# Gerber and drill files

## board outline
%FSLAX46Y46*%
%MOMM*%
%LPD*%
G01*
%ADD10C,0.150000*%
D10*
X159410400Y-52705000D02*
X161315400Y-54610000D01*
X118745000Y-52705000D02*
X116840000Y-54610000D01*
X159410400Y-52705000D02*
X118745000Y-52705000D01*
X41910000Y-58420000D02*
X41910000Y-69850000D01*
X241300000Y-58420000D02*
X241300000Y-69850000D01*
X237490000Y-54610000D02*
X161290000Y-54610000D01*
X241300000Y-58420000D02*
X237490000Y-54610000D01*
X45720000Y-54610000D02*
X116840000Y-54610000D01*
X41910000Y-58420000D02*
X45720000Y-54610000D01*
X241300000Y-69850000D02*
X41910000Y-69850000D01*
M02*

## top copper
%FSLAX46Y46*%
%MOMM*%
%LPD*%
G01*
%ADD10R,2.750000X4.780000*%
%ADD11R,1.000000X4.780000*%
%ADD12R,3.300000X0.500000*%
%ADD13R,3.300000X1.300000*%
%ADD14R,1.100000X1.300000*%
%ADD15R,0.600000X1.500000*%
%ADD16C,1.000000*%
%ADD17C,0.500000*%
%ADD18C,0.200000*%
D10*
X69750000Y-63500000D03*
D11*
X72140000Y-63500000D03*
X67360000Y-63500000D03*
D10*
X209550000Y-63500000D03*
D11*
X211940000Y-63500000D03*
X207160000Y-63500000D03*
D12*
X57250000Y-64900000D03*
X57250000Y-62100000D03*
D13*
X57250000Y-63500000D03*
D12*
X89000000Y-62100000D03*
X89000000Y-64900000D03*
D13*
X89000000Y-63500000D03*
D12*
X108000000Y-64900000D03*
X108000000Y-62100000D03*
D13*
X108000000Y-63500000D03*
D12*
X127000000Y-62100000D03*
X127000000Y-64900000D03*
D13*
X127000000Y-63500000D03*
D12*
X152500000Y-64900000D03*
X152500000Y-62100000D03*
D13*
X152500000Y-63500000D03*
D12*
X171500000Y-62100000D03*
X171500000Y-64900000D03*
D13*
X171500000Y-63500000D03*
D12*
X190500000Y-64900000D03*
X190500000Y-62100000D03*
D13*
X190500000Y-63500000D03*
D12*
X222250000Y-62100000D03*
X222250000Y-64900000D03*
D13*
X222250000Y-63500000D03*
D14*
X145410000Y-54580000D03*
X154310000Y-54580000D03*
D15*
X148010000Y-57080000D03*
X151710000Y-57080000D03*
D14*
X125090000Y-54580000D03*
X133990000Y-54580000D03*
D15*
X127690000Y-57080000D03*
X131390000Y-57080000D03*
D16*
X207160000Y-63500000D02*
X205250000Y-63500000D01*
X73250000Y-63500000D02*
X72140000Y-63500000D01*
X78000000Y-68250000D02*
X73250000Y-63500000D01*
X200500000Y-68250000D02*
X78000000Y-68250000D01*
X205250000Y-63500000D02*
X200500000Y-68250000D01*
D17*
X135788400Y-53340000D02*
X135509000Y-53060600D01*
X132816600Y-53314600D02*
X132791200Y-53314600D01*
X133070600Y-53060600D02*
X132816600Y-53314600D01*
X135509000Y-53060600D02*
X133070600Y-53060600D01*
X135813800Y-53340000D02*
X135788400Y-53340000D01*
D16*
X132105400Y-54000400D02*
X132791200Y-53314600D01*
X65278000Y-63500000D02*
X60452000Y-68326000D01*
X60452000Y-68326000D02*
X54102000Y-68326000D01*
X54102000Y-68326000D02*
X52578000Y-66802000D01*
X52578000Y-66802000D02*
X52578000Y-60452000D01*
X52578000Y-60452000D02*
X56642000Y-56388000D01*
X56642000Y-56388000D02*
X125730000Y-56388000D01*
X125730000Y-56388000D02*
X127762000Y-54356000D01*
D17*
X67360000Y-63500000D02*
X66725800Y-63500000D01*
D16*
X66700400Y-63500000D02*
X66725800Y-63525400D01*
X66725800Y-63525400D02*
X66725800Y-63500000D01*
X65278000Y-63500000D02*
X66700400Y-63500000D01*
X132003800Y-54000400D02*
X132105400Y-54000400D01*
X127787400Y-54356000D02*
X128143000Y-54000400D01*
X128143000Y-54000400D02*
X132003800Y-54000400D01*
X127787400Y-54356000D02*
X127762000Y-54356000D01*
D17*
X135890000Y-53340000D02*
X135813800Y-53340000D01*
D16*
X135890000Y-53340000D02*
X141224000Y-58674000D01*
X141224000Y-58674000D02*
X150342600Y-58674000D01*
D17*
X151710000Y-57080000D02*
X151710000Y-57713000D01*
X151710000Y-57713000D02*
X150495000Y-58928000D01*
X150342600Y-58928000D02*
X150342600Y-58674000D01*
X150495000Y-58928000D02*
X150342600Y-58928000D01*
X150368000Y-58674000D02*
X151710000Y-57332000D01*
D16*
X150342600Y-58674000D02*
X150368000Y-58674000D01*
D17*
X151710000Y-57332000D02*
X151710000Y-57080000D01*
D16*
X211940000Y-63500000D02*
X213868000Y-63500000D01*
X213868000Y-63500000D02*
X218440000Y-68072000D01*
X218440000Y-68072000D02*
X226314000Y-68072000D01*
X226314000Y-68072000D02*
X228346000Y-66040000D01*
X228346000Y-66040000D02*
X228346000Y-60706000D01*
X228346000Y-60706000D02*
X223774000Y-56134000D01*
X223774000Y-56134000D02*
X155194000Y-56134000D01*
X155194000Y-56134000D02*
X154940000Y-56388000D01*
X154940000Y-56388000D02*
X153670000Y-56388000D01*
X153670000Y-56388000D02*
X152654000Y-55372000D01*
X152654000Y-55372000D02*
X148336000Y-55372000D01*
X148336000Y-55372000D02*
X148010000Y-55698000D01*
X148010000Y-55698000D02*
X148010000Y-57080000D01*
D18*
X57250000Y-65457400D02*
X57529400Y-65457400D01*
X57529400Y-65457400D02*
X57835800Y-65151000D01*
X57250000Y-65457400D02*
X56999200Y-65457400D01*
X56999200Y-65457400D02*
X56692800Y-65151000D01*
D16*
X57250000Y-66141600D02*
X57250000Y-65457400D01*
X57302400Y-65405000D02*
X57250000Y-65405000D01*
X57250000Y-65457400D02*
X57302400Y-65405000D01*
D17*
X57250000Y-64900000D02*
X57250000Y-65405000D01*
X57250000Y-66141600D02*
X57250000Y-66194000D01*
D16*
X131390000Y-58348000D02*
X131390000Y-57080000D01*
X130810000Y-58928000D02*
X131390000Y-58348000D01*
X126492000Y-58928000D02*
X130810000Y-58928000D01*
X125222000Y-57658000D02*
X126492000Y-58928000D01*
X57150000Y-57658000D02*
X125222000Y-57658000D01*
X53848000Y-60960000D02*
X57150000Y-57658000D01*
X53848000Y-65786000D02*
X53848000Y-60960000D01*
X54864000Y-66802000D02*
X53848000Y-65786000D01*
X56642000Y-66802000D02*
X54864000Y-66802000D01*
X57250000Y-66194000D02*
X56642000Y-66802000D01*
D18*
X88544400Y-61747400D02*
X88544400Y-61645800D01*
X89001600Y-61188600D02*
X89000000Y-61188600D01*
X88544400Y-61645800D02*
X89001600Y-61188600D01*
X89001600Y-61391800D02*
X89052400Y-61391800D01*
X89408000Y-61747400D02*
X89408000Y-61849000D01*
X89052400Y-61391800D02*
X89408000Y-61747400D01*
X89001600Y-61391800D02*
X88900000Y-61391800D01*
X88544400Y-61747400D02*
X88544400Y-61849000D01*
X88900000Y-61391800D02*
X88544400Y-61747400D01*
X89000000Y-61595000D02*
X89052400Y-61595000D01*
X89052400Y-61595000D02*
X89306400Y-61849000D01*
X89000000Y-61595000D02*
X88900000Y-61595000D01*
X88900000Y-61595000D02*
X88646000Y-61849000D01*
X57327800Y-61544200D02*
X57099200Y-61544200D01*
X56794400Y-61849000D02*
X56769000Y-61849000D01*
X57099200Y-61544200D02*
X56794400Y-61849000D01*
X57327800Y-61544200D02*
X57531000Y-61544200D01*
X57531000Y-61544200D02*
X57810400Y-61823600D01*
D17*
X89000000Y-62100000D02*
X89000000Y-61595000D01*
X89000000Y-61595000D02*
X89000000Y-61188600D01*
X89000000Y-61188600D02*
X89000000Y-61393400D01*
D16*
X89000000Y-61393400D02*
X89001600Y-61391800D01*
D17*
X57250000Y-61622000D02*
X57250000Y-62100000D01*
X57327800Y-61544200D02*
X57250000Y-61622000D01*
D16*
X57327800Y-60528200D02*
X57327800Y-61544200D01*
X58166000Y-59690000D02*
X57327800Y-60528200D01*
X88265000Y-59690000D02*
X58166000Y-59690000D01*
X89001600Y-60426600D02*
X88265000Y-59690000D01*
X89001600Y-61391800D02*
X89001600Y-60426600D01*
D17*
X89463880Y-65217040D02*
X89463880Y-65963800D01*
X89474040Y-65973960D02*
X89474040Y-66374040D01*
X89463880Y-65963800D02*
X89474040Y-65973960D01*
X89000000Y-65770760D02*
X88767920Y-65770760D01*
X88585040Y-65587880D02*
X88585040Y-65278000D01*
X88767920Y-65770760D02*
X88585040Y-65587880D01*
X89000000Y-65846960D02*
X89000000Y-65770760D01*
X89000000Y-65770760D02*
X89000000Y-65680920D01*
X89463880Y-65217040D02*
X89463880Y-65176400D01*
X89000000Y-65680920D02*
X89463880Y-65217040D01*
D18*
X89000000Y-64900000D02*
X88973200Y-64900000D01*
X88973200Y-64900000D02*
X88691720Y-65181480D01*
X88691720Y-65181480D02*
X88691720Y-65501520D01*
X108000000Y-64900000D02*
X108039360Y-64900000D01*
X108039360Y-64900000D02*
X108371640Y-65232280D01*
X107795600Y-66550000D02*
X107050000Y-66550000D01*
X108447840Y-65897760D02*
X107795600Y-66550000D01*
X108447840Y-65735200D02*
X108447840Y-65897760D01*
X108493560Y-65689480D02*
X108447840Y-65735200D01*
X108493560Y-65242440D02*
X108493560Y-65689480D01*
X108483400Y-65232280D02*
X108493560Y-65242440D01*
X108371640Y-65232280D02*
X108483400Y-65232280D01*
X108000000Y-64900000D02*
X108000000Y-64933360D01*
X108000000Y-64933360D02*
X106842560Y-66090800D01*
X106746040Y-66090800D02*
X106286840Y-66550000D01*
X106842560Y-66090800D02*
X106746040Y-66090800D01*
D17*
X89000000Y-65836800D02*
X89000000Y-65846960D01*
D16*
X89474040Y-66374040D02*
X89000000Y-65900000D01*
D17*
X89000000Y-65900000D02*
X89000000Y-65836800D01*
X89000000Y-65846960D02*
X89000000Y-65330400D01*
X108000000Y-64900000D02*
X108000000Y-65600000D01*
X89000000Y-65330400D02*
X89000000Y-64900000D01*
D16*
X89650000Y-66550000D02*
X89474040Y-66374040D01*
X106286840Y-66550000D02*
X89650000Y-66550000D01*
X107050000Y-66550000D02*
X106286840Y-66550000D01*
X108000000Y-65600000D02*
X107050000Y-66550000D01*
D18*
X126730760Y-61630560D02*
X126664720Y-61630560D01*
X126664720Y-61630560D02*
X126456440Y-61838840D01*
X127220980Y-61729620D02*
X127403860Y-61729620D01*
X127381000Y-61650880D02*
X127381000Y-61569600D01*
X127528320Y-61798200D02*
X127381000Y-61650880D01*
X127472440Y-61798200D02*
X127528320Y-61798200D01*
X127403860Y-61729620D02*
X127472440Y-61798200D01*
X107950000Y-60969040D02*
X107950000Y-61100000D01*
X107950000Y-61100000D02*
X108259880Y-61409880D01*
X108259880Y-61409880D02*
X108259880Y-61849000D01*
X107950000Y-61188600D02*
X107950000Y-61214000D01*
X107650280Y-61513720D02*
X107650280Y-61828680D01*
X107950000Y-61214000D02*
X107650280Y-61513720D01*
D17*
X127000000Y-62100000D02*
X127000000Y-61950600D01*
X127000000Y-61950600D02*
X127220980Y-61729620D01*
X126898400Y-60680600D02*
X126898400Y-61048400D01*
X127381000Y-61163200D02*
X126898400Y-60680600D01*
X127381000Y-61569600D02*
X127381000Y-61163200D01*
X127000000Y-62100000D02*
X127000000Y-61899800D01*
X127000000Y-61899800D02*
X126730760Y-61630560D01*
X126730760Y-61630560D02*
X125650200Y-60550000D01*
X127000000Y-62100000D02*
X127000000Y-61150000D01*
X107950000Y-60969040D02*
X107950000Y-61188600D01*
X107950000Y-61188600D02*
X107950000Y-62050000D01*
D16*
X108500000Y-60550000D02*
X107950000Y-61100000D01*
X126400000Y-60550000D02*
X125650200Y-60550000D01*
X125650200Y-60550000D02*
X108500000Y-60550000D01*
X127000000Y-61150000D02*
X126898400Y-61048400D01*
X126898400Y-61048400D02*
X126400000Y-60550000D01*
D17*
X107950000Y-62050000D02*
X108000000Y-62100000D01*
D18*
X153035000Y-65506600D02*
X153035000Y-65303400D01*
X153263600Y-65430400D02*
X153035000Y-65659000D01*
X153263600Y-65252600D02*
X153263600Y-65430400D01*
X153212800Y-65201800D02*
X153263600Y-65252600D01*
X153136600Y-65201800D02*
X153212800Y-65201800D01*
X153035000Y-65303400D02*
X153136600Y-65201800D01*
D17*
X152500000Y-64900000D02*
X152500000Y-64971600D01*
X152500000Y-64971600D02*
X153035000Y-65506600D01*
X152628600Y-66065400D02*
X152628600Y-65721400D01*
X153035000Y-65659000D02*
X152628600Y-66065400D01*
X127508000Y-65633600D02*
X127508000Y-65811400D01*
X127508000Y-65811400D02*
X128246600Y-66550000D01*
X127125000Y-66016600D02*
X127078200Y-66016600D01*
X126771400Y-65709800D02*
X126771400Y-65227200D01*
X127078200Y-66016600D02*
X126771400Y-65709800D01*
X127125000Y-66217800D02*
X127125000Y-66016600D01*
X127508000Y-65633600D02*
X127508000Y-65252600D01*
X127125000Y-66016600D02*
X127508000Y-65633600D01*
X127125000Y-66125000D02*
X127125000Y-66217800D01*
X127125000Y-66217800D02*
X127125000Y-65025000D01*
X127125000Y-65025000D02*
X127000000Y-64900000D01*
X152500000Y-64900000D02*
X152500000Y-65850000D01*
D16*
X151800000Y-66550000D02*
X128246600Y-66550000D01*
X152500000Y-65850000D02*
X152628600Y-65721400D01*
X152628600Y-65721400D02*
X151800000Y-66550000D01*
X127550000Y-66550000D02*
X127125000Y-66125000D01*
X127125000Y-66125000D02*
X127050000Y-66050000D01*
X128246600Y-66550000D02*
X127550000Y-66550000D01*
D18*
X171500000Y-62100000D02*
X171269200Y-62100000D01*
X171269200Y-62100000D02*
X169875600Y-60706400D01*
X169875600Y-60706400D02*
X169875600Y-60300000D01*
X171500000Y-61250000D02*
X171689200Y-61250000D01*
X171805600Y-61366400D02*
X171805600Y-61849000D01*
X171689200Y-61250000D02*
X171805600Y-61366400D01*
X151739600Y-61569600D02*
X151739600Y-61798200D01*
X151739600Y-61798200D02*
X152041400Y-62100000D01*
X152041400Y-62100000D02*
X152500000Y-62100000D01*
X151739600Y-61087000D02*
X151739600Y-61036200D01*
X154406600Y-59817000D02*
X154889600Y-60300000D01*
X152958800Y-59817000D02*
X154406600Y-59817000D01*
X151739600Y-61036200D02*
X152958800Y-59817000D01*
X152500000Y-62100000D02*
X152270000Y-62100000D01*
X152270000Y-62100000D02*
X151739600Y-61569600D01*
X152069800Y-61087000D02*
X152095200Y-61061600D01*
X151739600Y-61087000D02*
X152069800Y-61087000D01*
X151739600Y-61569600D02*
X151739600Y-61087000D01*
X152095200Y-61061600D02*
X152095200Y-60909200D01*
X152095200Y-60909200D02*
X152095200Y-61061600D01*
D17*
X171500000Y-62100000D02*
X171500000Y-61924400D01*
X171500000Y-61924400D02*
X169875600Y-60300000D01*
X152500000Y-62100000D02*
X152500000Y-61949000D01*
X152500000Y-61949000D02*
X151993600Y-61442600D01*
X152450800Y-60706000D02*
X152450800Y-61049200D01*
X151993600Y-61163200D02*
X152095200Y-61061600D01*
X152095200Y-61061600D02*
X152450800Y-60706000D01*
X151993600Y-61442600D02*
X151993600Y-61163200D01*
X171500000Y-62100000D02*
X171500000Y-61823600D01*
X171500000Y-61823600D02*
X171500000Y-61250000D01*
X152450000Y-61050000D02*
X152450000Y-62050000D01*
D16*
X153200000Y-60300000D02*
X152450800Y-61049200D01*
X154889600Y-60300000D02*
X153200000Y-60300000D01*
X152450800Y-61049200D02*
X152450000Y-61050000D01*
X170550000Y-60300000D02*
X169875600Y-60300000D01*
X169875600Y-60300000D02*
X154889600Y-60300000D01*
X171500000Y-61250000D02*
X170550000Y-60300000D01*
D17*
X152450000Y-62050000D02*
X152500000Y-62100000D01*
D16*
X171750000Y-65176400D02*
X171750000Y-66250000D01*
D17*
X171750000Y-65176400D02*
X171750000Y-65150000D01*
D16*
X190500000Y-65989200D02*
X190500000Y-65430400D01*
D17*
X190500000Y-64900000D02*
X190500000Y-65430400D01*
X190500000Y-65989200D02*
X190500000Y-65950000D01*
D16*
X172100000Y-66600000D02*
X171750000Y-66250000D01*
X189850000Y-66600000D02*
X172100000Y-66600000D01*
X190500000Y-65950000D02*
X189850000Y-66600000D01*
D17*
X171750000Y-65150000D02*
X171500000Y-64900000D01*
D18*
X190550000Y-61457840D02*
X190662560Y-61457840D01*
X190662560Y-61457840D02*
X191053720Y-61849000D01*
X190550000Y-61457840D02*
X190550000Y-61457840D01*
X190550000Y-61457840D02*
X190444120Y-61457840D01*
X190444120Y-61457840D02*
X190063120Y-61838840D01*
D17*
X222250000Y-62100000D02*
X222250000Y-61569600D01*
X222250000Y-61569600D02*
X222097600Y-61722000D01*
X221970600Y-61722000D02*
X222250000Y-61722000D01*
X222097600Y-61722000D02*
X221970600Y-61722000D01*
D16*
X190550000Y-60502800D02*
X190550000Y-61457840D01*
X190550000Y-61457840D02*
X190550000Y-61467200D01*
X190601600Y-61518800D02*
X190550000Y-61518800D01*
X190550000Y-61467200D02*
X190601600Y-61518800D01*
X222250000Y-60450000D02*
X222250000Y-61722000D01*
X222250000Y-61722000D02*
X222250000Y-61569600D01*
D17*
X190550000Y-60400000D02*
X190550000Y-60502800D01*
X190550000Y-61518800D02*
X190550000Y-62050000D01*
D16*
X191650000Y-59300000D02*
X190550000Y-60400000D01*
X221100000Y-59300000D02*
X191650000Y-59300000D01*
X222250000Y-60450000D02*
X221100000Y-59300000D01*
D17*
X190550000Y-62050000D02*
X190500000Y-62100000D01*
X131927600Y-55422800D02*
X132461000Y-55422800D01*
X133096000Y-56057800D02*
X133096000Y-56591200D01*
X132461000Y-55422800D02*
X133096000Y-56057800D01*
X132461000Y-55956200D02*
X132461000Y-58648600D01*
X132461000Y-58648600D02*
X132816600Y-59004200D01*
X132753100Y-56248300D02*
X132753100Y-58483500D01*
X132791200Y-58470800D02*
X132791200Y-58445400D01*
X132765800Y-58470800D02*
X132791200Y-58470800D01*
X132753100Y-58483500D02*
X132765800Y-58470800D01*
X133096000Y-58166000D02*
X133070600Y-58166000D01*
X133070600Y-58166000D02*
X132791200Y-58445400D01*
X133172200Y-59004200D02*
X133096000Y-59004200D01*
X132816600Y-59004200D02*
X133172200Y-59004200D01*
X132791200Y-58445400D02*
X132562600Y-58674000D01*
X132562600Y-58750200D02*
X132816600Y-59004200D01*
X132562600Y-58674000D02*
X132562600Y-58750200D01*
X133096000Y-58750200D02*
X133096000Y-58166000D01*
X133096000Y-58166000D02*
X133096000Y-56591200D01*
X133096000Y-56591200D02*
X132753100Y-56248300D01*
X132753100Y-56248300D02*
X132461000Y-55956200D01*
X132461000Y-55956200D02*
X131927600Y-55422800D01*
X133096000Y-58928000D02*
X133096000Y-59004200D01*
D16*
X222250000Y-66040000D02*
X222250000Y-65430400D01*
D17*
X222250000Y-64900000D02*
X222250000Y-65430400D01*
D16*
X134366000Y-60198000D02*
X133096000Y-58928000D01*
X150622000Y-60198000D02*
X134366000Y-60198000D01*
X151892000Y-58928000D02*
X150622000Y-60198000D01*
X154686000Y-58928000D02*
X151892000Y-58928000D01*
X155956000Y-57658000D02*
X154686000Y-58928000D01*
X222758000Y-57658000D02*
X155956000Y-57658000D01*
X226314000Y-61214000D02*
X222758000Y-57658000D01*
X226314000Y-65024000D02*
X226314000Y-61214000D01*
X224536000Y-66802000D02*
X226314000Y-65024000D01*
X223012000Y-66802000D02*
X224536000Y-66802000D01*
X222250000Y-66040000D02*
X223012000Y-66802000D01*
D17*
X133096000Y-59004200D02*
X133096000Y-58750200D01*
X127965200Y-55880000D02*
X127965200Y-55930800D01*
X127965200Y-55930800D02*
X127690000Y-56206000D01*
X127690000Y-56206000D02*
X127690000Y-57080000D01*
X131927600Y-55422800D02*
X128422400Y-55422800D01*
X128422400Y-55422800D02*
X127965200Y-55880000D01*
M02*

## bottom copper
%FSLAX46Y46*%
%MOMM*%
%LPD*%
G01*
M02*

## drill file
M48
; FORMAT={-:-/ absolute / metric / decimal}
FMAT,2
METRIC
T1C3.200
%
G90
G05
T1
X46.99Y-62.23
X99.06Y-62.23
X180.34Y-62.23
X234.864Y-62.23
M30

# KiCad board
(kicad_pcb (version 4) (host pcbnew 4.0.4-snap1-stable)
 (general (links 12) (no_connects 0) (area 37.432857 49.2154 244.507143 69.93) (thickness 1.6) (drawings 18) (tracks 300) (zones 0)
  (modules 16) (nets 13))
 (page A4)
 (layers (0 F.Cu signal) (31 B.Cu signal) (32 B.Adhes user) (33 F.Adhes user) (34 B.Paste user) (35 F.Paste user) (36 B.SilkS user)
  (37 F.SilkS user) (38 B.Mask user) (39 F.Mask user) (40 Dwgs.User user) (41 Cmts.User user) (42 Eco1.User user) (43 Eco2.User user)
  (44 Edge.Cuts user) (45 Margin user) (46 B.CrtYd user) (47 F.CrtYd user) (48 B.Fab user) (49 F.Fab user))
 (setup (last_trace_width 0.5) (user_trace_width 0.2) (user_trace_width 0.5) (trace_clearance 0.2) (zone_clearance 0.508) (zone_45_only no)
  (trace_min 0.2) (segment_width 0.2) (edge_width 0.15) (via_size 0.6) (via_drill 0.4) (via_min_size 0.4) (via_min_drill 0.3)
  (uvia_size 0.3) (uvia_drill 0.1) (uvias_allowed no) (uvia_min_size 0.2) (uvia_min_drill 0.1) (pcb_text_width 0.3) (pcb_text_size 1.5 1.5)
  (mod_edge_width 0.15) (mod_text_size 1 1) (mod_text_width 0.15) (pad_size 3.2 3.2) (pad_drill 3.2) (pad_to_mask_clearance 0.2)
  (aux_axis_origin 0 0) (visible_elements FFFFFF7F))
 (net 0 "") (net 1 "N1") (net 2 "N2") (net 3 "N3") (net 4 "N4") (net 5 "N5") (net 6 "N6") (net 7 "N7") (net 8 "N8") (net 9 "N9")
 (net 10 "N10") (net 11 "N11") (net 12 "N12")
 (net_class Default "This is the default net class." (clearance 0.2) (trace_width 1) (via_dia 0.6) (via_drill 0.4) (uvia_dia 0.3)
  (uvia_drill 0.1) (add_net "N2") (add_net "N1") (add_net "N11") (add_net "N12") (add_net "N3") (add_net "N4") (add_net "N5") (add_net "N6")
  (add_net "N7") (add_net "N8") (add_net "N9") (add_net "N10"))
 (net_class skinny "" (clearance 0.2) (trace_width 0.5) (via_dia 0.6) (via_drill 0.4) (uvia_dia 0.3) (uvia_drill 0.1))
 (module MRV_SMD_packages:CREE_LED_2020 (layer F.Cu) (at 69.75 63.5 180)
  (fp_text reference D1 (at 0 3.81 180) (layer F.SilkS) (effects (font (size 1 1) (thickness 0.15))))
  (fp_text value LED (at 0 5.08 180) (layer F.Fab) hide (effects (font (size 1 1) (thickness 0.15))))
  (pad 0 smd rect (at 0 0 180) (size 2.75 4.78) (layers F.Cu F.Mask) (solder_mask_margin -5))
  (pad 2 smd rect (at -2.39 0 180) (size 1 4.78) (layers F.Cu F.Paste F.Mask) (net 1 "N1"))
  (pad 1 smd rect (at 2.39 0 180) (size 1 4.78) (layers F.Cu F.Paste F.Mask) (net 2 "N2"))
  (pad 0 smd rect (at -0.61 -0.525 180) (size 0.97 0.8) (layers F.Paste F.Mask))
  (pad 0 smd rect (at -0.61 -1.575 180) (size 0.97 0.8) (layers F.Paste F.Mask))
  (pad 0 smd rect (at 0.61 -1.575 180) (size 0.97 0.8) (layers F.Paste F.Mask))
  (pad 0 smd rect (at 0.61 -0.525 180) (size 0.97 0.8) (layers F.Paste F.Mask))
  (pad 0 smd rect (at 0.61 0.525 180) (size 0.97 0.8) (layers F.Paste F.Mask))
  (pad 0 smd rect (at -0.61 0.525 180) (size 0.97 0.8) (layers F.Paste F.Mask))
  (pad 0 smd rect (at -0.61 1.575 180) (size 0.97 0.8) (layers F.Paste F.Mask))
  (pad 0 smd rect (at 0.61 1.575 180) (size 0.97 0.8) (layers F.Paste F.Mask)))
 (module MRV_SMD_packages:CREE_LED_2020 (layer F.Cu) (at 209.55 63.5 180)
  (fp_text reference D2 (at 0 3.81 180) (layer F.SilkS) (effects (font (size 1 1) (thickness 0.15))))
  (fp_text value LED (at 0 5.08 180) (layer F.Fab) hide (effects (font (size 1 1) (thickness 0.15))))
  (pad 0 smd rect (at 0 0 180) (size 2.75 4.78) (layers F.Cu F.Mask) (solder_mask_margin -5))
  (pad 2 smd rect (at -2.39 0 180) (size 1 4.78) (layers F.Cu F.Paste F.Mask) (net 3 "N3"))
  (pad 1 smd rect (at 2.39 0 180) (size 1 4.78) (layers F.Cu F.Paste F.Mask) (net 1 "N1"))
  (pad 0 smd rect (at -0.61 -0.525 180) (size 0.97 0.8) (layers F.Paste F.Mask))
  (pad 0 smd rect (at -0.61 -1.575 180) (size 0.97 0.8) (layers F.Paste F.Mask))
  (pad 0 smd rect (at 0.61 -1.575 180) (size 0.97 0.8) (layers F.Paste F.Mask))
  (pad 0 smd rect (at 0.61 -0.525 180) (size 0.97 0.8) (layers F.Paste F.Mask))
  (pad 0 smd rect (at 0.61 0.525 180) (size 0.97 0.8) (layers F.Paste F.Mask))
  (pad 0 smd rect (at -0.61 0.525 180) (size 0.97 0.8) (layers F.Paste F.Mask))
  (pad 0 smd rect (at -0.61 1.575 180) (size 0.97 0.8) (layers F.Paste F.Mask))
  (pad 0 smd rect (at 0.61 1.575 180) (size 0.97 0.8) (layers F.Paste F.Mask)))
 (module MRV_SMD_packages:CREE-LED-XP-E (layer F.Cu) (at 57.25 63.5 270)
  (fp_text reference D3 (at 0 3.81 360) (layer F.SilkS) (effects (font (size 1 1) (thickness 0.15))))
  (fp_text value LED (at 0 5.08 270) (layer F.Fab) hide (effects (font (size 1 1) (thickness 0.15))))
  (pad 1 smd rect (at 1.4 0 270) (size 0.5 3.3) (layers F.Cu F.Paste F.Mask) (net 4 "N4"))
  (pad 2 smd rect (at -1.4 0 270) (size 0.5 3.3) (layers F.Cu F.Paste F.Mask) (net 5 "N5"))
  (pad 0 smd rect (at 0 0 270) (size 1.3 3.3) (layers F.Cu F.Paste F.Mask)))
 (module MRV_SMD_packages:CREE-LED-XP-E (layer F.Cu) (at 89 63.5 90)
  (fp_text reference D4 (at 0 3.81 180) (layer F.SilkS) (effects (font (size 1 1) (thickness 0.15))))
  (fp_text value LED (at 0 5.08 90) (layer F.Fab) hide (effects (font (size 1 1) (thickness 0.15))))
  (pad 1 smd rect (at 1.4 0 90) (size 0.5 3.3) (layers F.Cu F.Paste F.Mask) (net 5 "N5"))
  (pad 2 smd rect (at -1.4 0 90) (size 0.5 3.3) (layers F.Cu F.Paste F.Mask) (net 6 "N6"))
  (pad 0 smd rect (at 0 0 90) (size 1.3 3.3) (layers F.Cu F.Paste F.Mask)))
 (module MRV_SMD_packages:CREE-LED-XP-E (layer F.Cu) (at 108 63.5 270)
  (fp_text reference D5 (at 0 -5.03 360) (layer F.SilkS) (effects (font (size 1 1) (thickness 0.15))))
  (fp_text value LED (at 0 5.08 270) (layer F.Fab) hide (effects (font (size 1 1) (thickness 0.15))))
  (pad 1 smd rect (at 1.4 0 270) (size 0.5 3.3) (layers F.Cu F.Paste F.Mask) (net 6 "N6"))
  (pad 2 smd rect (at -1.4 0 270) (size 0.5 3.3) (layers F.Cu F.Paste F.Mask) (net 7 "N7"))
  (pad 0 smd rect (at 0 0 270) (size 1.3 3.3) (layers F.Cu F.Paste F.Mask)))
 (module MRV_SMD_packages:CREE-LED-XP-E (layer F.Cu) (at 127 63.5 90)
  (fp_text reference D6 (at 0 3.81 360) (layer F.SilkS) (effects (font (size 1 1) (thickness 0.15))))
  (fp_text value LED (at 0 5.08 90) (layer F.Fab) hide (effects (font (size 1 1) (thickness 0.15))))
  (pad 1 smd rect (at 1.4 0 90) (size 0.5 3.3) (layers F.Cu F.Paste F.Mask) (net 7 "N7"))
  (pad 2 smd rect (at -1.4 0 90) (size 0.5 3.3) (layers F.Cu F.Paste F.Mask) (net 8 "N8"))
  (pad 0 smd rect (at 0 0 90) (size 1.3 3.3) (layers F.Cu F.Paste F.Mask)))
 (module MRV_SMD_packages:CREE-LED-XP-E (layer F.Cu) (at 152.5 63.5 270)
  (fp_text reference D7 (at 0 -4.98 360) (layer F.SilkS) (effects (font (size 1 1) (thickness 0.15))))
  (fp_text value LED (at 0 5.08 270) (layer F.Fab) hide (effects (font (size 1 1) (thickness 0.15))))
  (pad 1 smd rect (at 1.4 0 270) (size 0.5 3.3) (layers F.Cu F.Paste F.Mask) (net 8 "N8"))
  (pad 2 smd rect (at -1.4 0 270) (size 0.5 3.3) (layers F.Cu F.Paste F.Mask) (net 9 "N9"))
  (pad 0 smd rect (at 0 0 270) (size 1.3 3.3) (layers F.Cu F.Paste F.Mask)))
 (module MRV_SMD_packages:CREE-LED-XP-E (layer F.Cu) (at 171.5 63.5 90)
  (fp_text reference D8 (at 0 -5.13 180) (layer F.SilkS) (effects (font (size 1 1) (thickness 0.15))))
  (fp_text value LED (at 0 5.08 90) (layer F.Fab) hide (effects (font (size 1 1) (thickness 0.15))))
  (pad 1 smd rect (at 1.4 0 90) (size 0.5 3.3) (layers F.Cu F.Paste F.Mask) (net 9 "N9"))
  (pad 2 smd rect (at -1.4 0 90) (size 0.5 3.3) (layers F.Cu F.Paste F.Mask) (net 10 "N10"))
  (pad 0 smd rect (at 0 0 90) (size 1.3 3.3) (layers F.Cu F.Paste F.Mask)))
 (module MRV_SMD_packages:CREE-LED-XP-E (layer F.Cu) (at 190.5 63.5 270)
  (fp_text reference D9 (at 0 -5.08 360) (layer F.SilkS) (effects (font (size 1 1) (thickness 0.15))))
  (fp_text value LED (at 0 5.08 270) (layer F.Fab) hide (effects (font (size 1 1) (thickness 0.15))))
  (pad 1 smd rect (at 1.4 0 270) (size 0.5 3.3) (layers F.Cu F.Paste F.Mask) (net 10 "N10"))
  (pad 2 smd rect (at -1.4 0 270) (size 0.5 3.3) (layers F.Cu F.Paste F.Mask) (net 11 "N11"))
  (pad 0 smd rect (at 0 0 270) (size 1.3 3.3) (layers F.Cu F.Paste F.Mask)))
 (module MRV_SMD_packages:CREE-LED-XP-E (layer F.Cu) (at 222.25 63.5 90)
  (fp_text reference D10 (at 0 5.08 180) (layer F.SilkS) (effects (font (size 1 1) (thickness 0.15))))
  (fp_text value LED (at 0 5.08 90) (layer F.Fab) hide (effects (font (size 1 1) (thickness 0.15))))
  (pad 1 smd rect (at 1.4 0 90) (size 0.5 3.3) (layers F.Cu F.Paste F.Mask) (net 11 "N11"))
  (pad 2 smd rect (at -1.4 0 90) (size 0.5 3.3) (layers F.Cu F.Paste F.Mask) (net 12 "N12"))
  (pad 0 smd rect (at 0 0 90) (size 1.3 3.3) (layers F.Cu F.Paste F.Mask)))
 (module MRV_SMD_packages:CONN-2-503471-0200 (layer F.Cu) (at 149.86 55.88 180)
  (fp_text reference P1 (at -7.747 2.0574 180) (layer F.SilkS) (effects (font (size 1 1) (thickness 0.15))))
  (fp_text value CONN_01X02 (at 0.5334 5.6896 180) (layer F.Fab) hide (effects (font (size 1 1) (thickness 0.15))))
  (pad 0 smd rect (at 4.45 1.3 180) (size 1.1 1.3) (layers F.Cu F.Paste F.Mask))
  (pad 0 smd rect (at -4.45 1.3 180) (size 1.1 1.3) (layers F.Cu F.Paste F.Mask))
  (pad 2 smd rect (at 1.85 -1.2 180) (size 0.6 1.5) (layers F.Cu F.Paste F.Mask) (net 3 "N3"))
  (pad 1 smd rect (at -1.85 -1.2 180) (size 0.6 1.5) (layers F.Cu F.Paste F.Mask) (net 2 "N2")))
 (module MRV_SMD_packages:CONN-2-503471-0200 (layer F.Cu) (at 129.54 55.88 180)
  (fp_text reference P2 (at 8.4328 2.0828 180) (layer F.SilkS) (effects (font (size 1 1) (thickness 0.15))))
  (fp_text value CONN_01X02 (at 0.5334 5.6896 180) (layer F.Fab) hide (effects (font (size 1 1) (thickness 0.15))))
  (pad 0 smd rect (at 4.45 1.3 180) (size 1.1 1.3) (layers F.Cu F.Paste F.Mask))
  (pad 0 smd rect (at -4.45 1.3 180) (size 1.1 1.3) (layers F.Cu F.Paste F.Mask))
  (pad 2 smd rect (at 1.85 -1.2 180) (size 0.6 1.5) (layers F.Cu F.Paste F.Mask) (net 12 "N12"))
  (pad 1 smd rect (at -1.85 -1.2 180) (size 0.6 1.5) (layers F.Cu F.Paste F.Mask) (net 4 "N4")))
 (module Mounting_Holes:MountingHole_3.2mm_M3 (layer F.Cu) (at 46.99 62.23)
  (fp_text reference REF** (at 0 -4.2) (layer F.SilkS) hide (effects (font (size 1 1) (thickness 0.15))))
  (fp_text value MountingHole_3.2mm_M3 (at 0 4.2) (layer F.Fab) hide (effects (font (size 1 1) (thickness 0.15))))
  (pad 1 np_thru_hole circle (at 0 0) (size 3.2 3.2) (drill 3.2) (layers *.Cu *.Mask F.SilkS)))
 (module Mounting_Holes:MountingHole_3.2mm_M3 (layer F.Cu) (at 234.86364 62.3062)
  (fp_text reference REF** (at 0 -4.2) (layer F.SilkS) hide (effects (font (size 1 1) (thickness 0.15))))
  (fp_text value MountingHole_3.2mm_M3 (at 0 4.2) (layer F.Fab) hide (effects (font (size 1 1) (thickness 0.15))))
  (pad "" np_thru_hole circle (at 0 -0.0762) (size 3.2 3.2) (drill 3.2) (layers *.Cu *.Mask F.SilkS)))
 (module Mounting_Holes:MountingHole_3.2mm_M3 (layer F.Cu) (at 180.34 62.23)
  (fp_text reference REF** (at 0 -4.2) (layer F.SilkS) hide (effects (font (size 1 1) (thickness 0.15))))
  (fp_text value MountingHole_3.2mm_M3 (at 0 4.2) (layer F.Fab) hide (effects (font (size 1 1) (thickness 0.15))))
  (pad 1 np_thru_hole circle (at 0 0) (size 3.2 3.2) (drill 3.2) (layers *.Cu *.Mask F.SilkS)))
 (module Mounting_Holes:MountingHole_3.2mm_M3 (layer F.Cu) (at 99.06 62.23)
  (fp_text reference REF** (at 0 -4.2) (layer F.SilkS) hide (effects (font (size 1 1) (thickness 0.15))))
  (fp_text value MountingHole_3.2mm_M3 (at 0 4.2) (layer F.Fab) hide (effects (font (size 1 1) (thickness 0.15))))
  (pad 1 np_thru_hole circle (at 0 0) (size 3.2 3.2) (drill 3.2) (layers *.Cu *.Mask F.SilkS)))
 (gr_line (start 159.4104 52.705) (end 161.3154 54.61) (angle 90) (layer Edge.Cuts) (width 0.15))
 (gr_line (start 118.745 52.705) (end 116.84 54.61) (angle 90) (layer Edge.Cuts) (width 0.15))
 (gr_line (start 159.4104 52.705) (end 118.745 52.705) (angle 90) (layer Edge.Cuts) (width 0.15))
 (gr_line (start 41.91 58.42) (end 41.91 69.85) (angle 90) (layer Edge.Cuts) (width 0.15))
 (gr_line (start 241.3 58.42) (end 241.3 69.85) (angle 90) (layer Edge.Cuts) (width 0.15))
 (gr_line (start 237.49 54.61) (end 161.29 54.61) (angle 90) (layer Edge.Cuts) (width 0.15))
 (gr_line (start 241.3 58.42) (end 237.49 54.61) (angle 90) (layer Edge.Cuts) (width 0.15))
 (gr_line (start 45.72 54.61) (end 116.84 54.61) (angle 90) (layer Edge.Cuts) (width 0.15))
 (gr_line (start 41.91 58.42) (end 45.72 54.61) (angle 90) (layer Edge.Cuts) (width 0.15))
 (gr_line (start 241.3 69.85) (end 41.91 69.85) (angle 90) (layer Edge.Cuts) (width 0.15))
 (segment (start 207.16 63.5) (end 205.25 63.5) (width 1) (layer F.Cu) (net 1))
 (segment (start 73.25 63.5) (end 72.14 63.5) (width 1) (layer F.Cu) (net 1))
 (segment (start 78 68.25) (end 73.25 63.5) (width 1) (layer F.Cu) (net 1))
 (segment (start 200.5 68.25) (end 78 68.25) (width 1) (layer F.Cu) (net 1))
 (segment (start 205.25 63.5) (end 200.5 68.25) (width 1) (layer F.Cu) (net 1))
 (segment (start 135.7884 53.34) (end 135.509 53.0606) (width 0.5) (layer F.Cu) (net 2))
 (segment (start 132.8166 53.3146) (end 132.7912 53.3146) (width 0.5) (layer F.Cu) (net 2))
 (segment (start 133.0706 53.0606) (end 132.8166 53.3146) (width 0.5) (layer F.Cu) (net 2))
 (segment (start 135.509 53.0606) (end 133.0706 53.0606) (width 0.5) (layer F.Cu) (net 2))
 (segment (start 135.8138 53.34) (end 135.7884 53.34) (width 0.5) (layer F.Cu) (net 2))
 (segment (start 132.1054 54.0004) (end 132.7912 53.3146) (width 1) (layer F.Cu) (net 2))
 (segment (start 65.278 63.5) (end 60.452 68.326) (width 1) (layer F.Cu) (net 2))
 (segment (start 60.452 68.326) (end 54.102 68.326) (width 1) (layer F.Cu) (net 2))
 (segment (start 54.102 68.326) (end 52.578 66.802) (width 1) (layer F.Cu) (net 2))
 (segment (start 52.578 66.802) (end 52.578 60.452) (width 1) (layer F.Cu) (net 2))
 (segment (start 52.578 60.452) (end 56.642 56.388) (width 1) (layer F.Cu) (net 2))
 (segment (start 56.642 56.388) (end 125.73 56.388) (width 1) (layer F.Cu) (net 2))
 (segment (start 125.73 56.388) (end 127.762 54.356) (width 1) (layer F.Cu) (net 2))
 (segment (start 67.36 63.5) (end 66.7258 63.5) (width 0.5) (layer F.Cu) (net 2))
 (segment (start 66.7004 63.5) (end 66.7258 63.5254) (width 1) (layer F.Cu) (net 2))
 (segment (start 66.7258 63.5254) (end 66.7258 63.5) (width 1) (layer F.Cu) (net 2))
 (segment (start 65.278 63.5) (end 66.7004 63.5) (width 1) (layer F.Cu) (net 2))
 (segment (start 132.0038 54.0004) (end 132.1054 54.0004) (width 1) (layer F.Cu) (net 2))
 (segment (start 127.7874 54.356) (end 128.143 54.0004) (width 1) (layer F.Cu) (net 2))
 (segment (start 128.143 54.0004) (end 132.0038 54.0004) (width 1) (layer F.Cu) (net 2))
 (segment (start 127.7874 54.356) (end 127.762 54.356) (width 1) (layer F.Cu) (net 2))
 (segment (start 135.89 53.34) (end 135.8138 53.34) (width 0.5) (layer F.Cu) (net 2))
 (segment (start 135.89 53.34) (end 141.224 58.674) (width 1) (layer F.Cu) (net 2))
 (segment (start 141.224 58.674) (end 150.3426 58.674) (width 1) (layer F.Cu) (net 2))
 (segment (start 151.71 57.08) (end 151.71 57.713) (width 0.5) (layer F.Cu) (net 2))
 (segment (start 151.71 57.713) (end 150.495 58.928) (width 0.5) (layer F.Cu) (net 2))
 (segment (start 150.3426 58.928) (end 150.3426 58.674) (width 0.5) (layer F.Cu) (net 2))
 (segment (start 150.495 58.928) (end 150.3426 58.928) (width 0.5) (layer F.Cu) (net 2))
 (segment (start 150.368 58.674) (end 151.71 57.332) (width 0.5) (layer F.Cu) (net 2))
 (segment (start 150.3426 58.674) (end 150.368 58.674) (width 1) (layer F.Cu) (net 2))
 (segment (start 151.71 57.332) (end 151.71 57.08) (width 0.5) (layer F.Cu) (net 2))
 (segment (start 211.94 63.5) (end 213.868 63.5) (width 1) (layer F.Cu) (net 3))
 (segment (start 213.868 63.5) (end 218.44 68.072) (width 1) (layer F.Cu) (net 3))
 (segment (start 218.44 68.072) (end 226.314 68.072) (width 1) (layer F.Cu) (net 3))
 (segment (start 226.314 68.072) (end 228.346 66.04) (width 1) (layer F.Cu) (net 3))
 (segment (start 228.346 66.04) (end 228.346 60.706) (width 1) (layer F.Cu) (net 3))
 (segment (start 228.346 60.706) (end 223.774 56.134) (width 1) (layer F.Cu) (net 3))
 (segment (start 223.774 56.134) (end 155.194 56.134) (width 1) (layer F.Cu) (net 3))
 (segment (start 155.194 56.134) (end 154.94 56.388) (width 1) (layer F.Cu) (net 3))
 (segment (start 154.94 56.388) (end 153.67 56.388) (width 1) (layer F.Cu) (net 3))
 (segment (start 153.67 56.388) (end 152.654 55.372) (width 1) (layer F.Cu) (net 3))
 (segment (start 152.654 55.372) (end 148.336 55.372) (width 1) (layer F.Cu) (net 3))
 (segment (start 148.336 55.372) (end 148.01 55.698) (width 1) (layer F.Cu) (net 3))
 (segment (start 148.01 55.698) (end 148.01 57.08) (width 1) (layer F.Cu) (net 3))
 (segment (start 57.25 65.4574) (end 57.5294 65.4574) (width 0.2) (layer F.Cu) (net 4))
 (segment (start 57.5294 65.4574) (end 57.8358 65.151) (width 0.2) (layer F.Cu) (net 4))
 (segment (start 57.25 65.4574) (end 56.9992 65.4574) (width 0.2) (layer F.Cu) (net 4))
 (segment (start 56.9992 65.4574) (end 56.6928 65.151) (width 0.2) (layer F.Cu) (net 4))
 (segment (start 57.25 66.1416) (end 57.25 65.4574) (width 1) (layer F.Cu) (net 4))
 (segment (start 57.3024 65.405) (end 57.25 65.405) (width 1) (layer F.Cu) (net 4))
 (segment (start 57.25 65.4574) (end 57.3024 65.405) (width 1) (layer F.Cu) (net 4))
 (segment (start 57.25 64.9) (end 57.25 65.405) (width 0.5) (layer F.Cu) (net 4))
 (segment (start 57.25 66.1416) (end 57.25 66.194) (width 0.5) (layer F.Cu) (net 4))
 (segment (start 131.39 58.348) (end 131.39 57.08) (width 1) (layer F.Cu) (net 4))
 (segment (start 130.81 58.928) (end 131.39 58.348) (width 1) (layer F.Cu) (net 4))
 (segment (start 126.492 58.928) (end 130.81 58.928) (width 1) (layer F.Cu) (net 4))
 (segment (start 125.222 57.658) (end 126.492 58.928) (width 1) (layer F.Cu) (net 4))
 (segment (start 57.15 57.658) (end 125.222 57.658) (width 1) (layer F.Cu) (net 4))
 (segment (start 53.848 60.96) (end 57.15 57.658) (width 1) (layer F.Cu) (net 4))
 (segment (start 53.848 65.786) (end 53.848 60.96) (width 1) (layer F.Cu) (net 4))
 (segment (start 54.864 66.802) (end 53.848 65.786) (width 1) (layer F.Cu) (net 4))
 (segment (start 56.642 66.802) (end 54.864 66.802) (width 1) (layer F.Cu) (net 4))
 (segment (start 57.25 66.194) (end 56.642 66.802) (width 1) (layer F.Cu) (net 4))
 (segment (start 88.5444 61.7474) (end 88.5444 61.6458) (width 0.2) (layer F.Cu) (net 5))
 (segment (start 89.0016 61.1886) (end 89 61.1886) (width 0.2) (layer F.Cu) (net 5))
 (segment (start 88.5444 61.6458) (end 89.0016 61.1886) (width 0.2) (layer F.Cu) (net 5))
 (segment (start 89.0016 61.3918) (end 89.0524 61.3918) (width 0.2) (layer F.Cu) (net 5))
 (segment (start 89.408 61.7474) (end 89.408 61.849) (width 0.2) (layer F.Cu) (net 5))
 (segment (start 89.0524 61.3918) (end 89.408 61.7474) (width 0.2) (layer F.Cu) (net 5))
 (segment (start 89.0016 61.3918) (end 88.9 61.3918) (width 0.2) (layer F.Cu) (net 5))
 (segment (start 88.5444 61.7474) (end 88.5444 61.849) (width 0.2) (layer F.Cu) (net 5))
 (segment (start 88.9 61.3918) (end 88.5444 61.7474) (width 0.2) (layer F.Cu) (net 5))
 (segment (start 89 61.595) (end 89.0524 61.595) (width 0.2) (layer F.Cu) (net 5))
 (segment (start 89.0524 61.595) (end 89.3064 61.849) (width 0.2) (layer F.Cu) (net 5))
 (segment (start 89 61.595) (end 88.9 61.595) (width 0.2) (layer F.Cu) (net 5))
 (segment (start 88.9 61.595) (end 88.646 61.849) (width 0.2) (layer F.Cu) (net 5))
 (segment (start 57.3278 61.5442) (end 57.0992 61.5442) (width 0.2) (layer F.Cu) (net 5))
 (segment (start 56.7944 61.849) (end 56.769 61.849) (width 0.2) (layer F.Cu) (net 5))
 (segment (start 57.0992 61.5442) (end 56.7944 61.849) (width 0.2) (layer F.Cu) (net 5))
 (segment (start 57.3278 61.5442) (end 57.531 61.5442) (width 0.2) (layer F.Cu) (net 5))
 (segment (start 57.531 61.5442) (end 57.8104 61.8236) (width 0.2) (layer F.Cu) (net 5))
 (segment (start 89 62.1) (end 89 61.595) (width 0.5) (layer F.Cu) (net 5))
 (segment (start 89 61.595) (end 89 61.1886) (width 0.5) (layer F.Cu) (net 5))
 (segment (start 89 61.1886) (end 89 61.3934) (width 0.5) (layer F.Cu) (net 5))
 (segment (start 89 61.3934) (end 89.0016 61.3918) (width 1) (layer F.Cu) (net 5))
 (segment (start 57.25 61.622) (end 57.25 62.1) (width 0.5) (layer F.Cu) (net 5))
 (segment (start 57.3278 61.5442) (end 57.25 61.622) (width 0.5) (layer F.Cu) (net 5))
 (segment (start 57.3278 60.5282) (end 57.3278 61.5442) (width 1) (layer F.Cu) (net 5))
 (segment (start 58.166 59.69) (end 57.3278 60.5282) (width 1) (layer F.Cu) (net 5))
 (segment (start 88.265 59.69) (end 58.166 59.69) (width 1) (layer F.Cu) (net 5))
 (segment (start 89.0016 60.4266) (end 88.265 59.69) (width 1) (layer F.Cu) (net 5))
 (segment (start 89.0016 61.3918) (end 89.0016 60.4266) (width 1) (layer F.Cu) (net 5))
 (segment (start 89.46388 65.21704) (end 89.46388 65.9638) (width 0.5) (layer F.Cu) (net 6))
 (segment (start 89.47404 65.97396) (end 89.47404 66.37404) (width 0.5) (layer F.Cu) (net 6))
 (segment (start 89.46388 65.9638) (end 89.47404 65.97396) (width 0.5) (layer F.Cu) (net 6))
 (segment (start 89 65.77076) (end 88.76792 65.77076) (width 0.5) (layer F.Cu) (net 6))
 (segment (start 88.58504 65.58788) (end 88.58504 65.278) (width 0.5) (layer F.Cu) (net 6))
 (segment (start 88.76792 65.77076) (end 88.58504 65.58788) (width 0.5) (layer F.Cu) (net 6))
 (segment (start 89 65.84696) (end 89 65.77076) (width 0.5) (layer F.Cu) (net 6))
 (segment (start 89 65.77076) (end 89 65.68092) (width 0.5) (layer F.Cu) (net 6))
 (segment (start 89.46388 65.21704) (end 89.46388 65.1764) (width 0.5) (layer F.Cu) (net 6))
 (segment (start 89 65.68092) (end 89.46388 65.21704) (width 0.5) (layer F.Cu) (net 6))
 (segment (start 89 64.9) (end 88.9732 64.9) (width 0.2) (layer F.Cu) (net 6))
 (segment (start 88.9732 64.9) (end 88.69172 65.18148) (width 0.2) (layer F.Cu) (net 6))
 (segment (start 88.69172 65.18148) (end 88.69172 65.50152) (width 0.2) (layer F.Cu) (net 6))
 (segment (start 108 64.9) (end 108.03936 64.9) (width 0.2) (layer F.Cu) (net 6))
 (segment (start 108.03936 64.9) (end 108.37164 65.23228) (width 0.2) (layer F.Cu) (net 6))
 (segment (start 107.7956 66.55) (end 107.05 66.55) (width 0.2) (layer F.Cu) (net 6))
 (segment (start 108.44784 65.89776) (end 107.7956 66.55) (width 0.2) (layer F.Cu) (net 6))
 (segment (start 108.44784 65.7352) (end 108.44784 65.89776) (width 0.2) (layer F.Cu) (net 6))
 (segment (start 108.49356 65.68948) (end 108.44784 65.7352) (width 0.2) (layer F.Cu) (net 6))
 (segment (start 108.49356 65.24244) (end 108.49356 65.68948) (width 0.2) (layer F.Cu) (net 6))
 (segment (start 108.4834 65.23228) (end 108.49356 65.24244) (width 0.2) (layer F.Cu) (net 6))
 (segment (start 108.37164 65.23228) (end 108.4834 65.23228) (width 0.2) (layer F.Cu) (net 6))
 (segment (start 108 64.9) (end 108 64.93336) (width 0.2) (layer F.Cu) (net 6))
 (segment (start 108 64.93336) (end 106.84256 66.0908) (width 0.2) (layer F.Cu) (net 6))
 (segment (start 106.74604 66.0908) (end 106.28684 66.55) (width 0.2) (layer F.Cu) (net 6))
 (segment (start 106.84256 66.0908) (end 106.74604 66.0908) (width 0.2) (layer F.Cu) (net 6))
 (segment (start 89 65.8368) (end 89 65.84696) (width 0.5) (layer F.Cu) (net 6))
 (segment (start 89.47404 66.37404) (end 89 65.9) (width 1) (layer F.Cu) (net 6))
 (segment (start 89 65.9) (end 89 65.8368) (width 0.5) (layer F.Cu) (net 6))
 (segment (start 89 65.84696) (end 89 65.3304) (width 0.5) (layer F.Cu) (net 6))
 (segment (start 108 64.9) (end 108 65.6) (width 0.5) (layer F.Cu) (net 6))
 (segment (start 89 65.3304) (end 89 64.9) (width 0.5) (layer F.Cu) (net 6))
 (segment (start 89.65 66.55) (end 89.47404 66.37404) (width 1) (layer F.Cu) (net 6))
 (segment (start 106.28684 66.55) (end 89.65 66.55) (width 1) (layer F.Cu) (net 6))
 (segment (start 107.05 66.55) (end 106.28684 66.55) (width 1) (layer F.Cu) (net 6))
 (segment (start 108 65.6) (end 107.05 66.55) (width 1) (layer F.Cu) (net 6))
 (segment (start 126.73076 61.63056) (end 126.66472 61.63056) (width 0.2) (layer F.Cu) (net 7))
 (segment (start 126.66472 61.63056) (end 126.45644 61.83884) (width 0.2) (layer F.Cu) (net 7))
 (segment (start 127.22098 61.72962) (end 127.40386 61.72962) (width 0.2) (layer F.Cu) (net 7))
 (segment (start 127.381 61.65088) (end 127.381 61.5696) (width 0.2) (layer F.Cu) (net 7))
 (segment (start 127.52832 61.7982) (end 127.381 61.65088) (width 0.2) (layer F.Cu) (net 7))
 (segment (start 127.47244 61.7982) (end 127.52832 61.7982) (width 0.2) (layer F.Cu) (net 7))
 (segment (start 127.40386 61.72962) (end 127.47244 61.7982) (width 0.2) (layer F.Cu) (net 7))
 (segment (start 107.95 60.96904) (end 107.95 61.1) (width 0.2) (layer F.Cu) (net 7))
 (segment (start 107.95 61.1) (end 108.25988 61.40988) (width 0.2) (layer F.Cu) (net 7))
 (segment (start 108.25988 61.40988) (end 108.25988 61.849) (width 0.2) (layer F.Cu) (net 7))
 (segment (start 107.95 61.1886) (end 107.95 61.214) (width 0.2) (layer F.Cu) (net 7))
 (segment (start 107.65028 61.51372) (end 107.65028 61.82868) (width 0.2) (layer F.Cu) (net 7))
 (segment (start 107.95 61.214) (end 107.65028 61.51372) (width 0.2) (layer F.Cu) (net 7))
 (segment (start 127 62.1) (end 127 61.9506) (width 0.5) (layer F.Cu) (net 7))
 (segment (start 127 61.9506) (end 127.22098 61.72962) (width 0.5) (layer F.Cu) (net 7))
 (segment (start 126.8984 60.6806) (end 126.8984 61.0484) (width 0.5) (layer F.Cu) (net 7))
 (segment (start 127.381 61.1632) (end 126.8984 60.6806) (width 0.5) (layer F.Cu) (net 7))
 (segment (start 127.381 61.5696) (end 127.381 61.1632) (width 0.5) (layer F.Cu) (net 7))
 (segment (start 127 62.1) (end 127 61.8998) (width 0.5) (layer F.Cu) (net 7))
 (segment (start 127 61.8998) (end 126.73076 61.63056) (width 0.5) (layer F.Cu) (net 7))
 (segment (start 126.73076 61.63056) (end 125.6502 60.55) (width 0.5) (layer F.Cu) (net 7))
 (segment (start 127 62.1) (end 127 61.15) (width 0.5) (layer F.Cu) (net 7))
 (segment (start 107.95 60.96904) (end 107.95 61.1886) (width 0.5) (layer F.Cu) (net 7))
 (segment (start 107.95 61.1886) (end 107.95 62.05) (width 0.5) (layer F.Cu) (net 7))
 (segment (start 108.5 60.55) (end 107.95 61.1) (width 1) (layer F.Cu) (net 7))
 (segment (start 126.4 60.55) (end 125.6502 60.55) (width 1) (layer F.Cu) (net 7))
 (segment (start 125.6502 60.55) (end 108.5 60.55) (width 1) (layer F.Cu) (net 7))
 (segment (start 127 61.15) (end 126.8984 61.0484) (width 1) (layer F.Cu) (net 7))
 (segment (start 126.8984 61.0484) (end 126.4 60.55) (width 1) (layer F.Cu) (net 7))
 (segment (start 107.95 62.05) (end 108 62.1) (width 0.5) (layer F.Cu) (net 7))
 (segment (start 153.035 65.5066) (end 153.035 65.3034) (width 0.2) (layer F.Cu) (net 8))
 (segment (start 153.2636 65.4304) (end 153.035 65.659) (width 0.2) (layer F.Cu) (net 8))
 (segment (start 153.2636 65.2526) (end 153.2636 65.4304) (width 0.2) (layer F.Cu) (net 8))
 (segment (start 153.2128 65.2018) (end 153.2636 65.2526) (width 0.2) (layer F.Cu) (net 8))
 (segment (start 153.1366 65.2018) (end 153.2128 65.2018) (width 0.2) (layer F.Cu) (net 8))
 (segment (start 153.035 65.3034) (end 153.1366 65.2018) (width 0.2) (layer F.Cu) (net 8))
 (segment (start 152.5 64.9) (end 152.5 64.9716) (width 0.5) (layer F.Cu) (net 8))
 (segment (start 152.5 64.9716) (end 153.035 65.5066) (width 0.5) (layer F.Cu) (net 8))
 (segment (start 152.6286 66.0654) (end 152.6286 65.7214) (width 0.5) (layer F.Cu) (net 8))
 (segment (start 153.035 65.659) (end 152.6286 66.0654) (width 0.5) (layer F.Cu) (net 8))
 (segment (start 127.508 65.6336) (end 127.508 65.8114) (width 0.5) (layer F.Cu) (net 8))
 (segment (start 127.508 65.8114) (end 128.2466 66.55) (width 0.5) (layer F.Cu) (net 8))
 (segment (start 127.125 66.0166) (end 127.0782 66.0166) (width 0.5) (layer F.Cu) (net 8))
 (segment (start 126.7714 65.7098) (end 126.7714 65.2272) (width 0.5) (layer F.Cu) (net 8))
 (segment (start 127.0782 66.0166) (end 126.7714 65.7098) (width 0.5) (layer F.Cu) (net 8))
 (segment (start 127.125 66.2178) (end 127.125 66.0166) (width 0.5) (layer F.Cu) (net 8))
 (segment (start 127.508 65.6336) (end 127.508 65.2526) (width 0.5) (layer F.Cu) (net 8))
 (segment (start 127.125 66.0166) (end 127.508 65.6336) (width 0.5) (layer F.Cu) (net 8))
 (segment (start 127.125 66.125) (end 127.125 66.2178) (width 0.5) (layer F.Cu) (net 8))
 (segment (start 127.125 66.2178) (end 127.125 65.025) (width 0.5) (layer F.Cu) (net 8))
 (segment (start 127.125 65.025) (end 127 64.9) (width 0.5) (layer F.Cu) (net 8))
 (segment (start 152.5 64.9) (end 152.5 65.85) (width 0.5) (layer F.Cu) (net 8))
 (segment (start 151.8 66.55) (end 128.2466 66.55) (width 1) (layer F.Cu) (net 8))
 (segment (start 152.5 65.85) (end 152.6286 65.7214) (width 1) (layer F.Cu) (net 8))
 (segment (start 152.6286 65.7214) (end 151.8 66.55) (width 1) (layer F.Cu) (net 8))
 (segment (start 127.55 66.55) (end 127.125 66.125) (width 1) (layer F.Cu) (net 8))
 (segment (start 127.125 66.125) (end 127.05 66.05) (width 1) (layer F.Cu) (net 8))
 (segment (start 128.2466 66.55) (end 127.55 66.55) (width 1) (layer F.Cu) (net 8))
 (segment (start 171.5 62.1) (end 171.2692 62.1) (width 0.2) (layer F.Cu) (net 9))
 (segment (start 171.2692 62.1) (end 169.8756 60.7064) (width 0.2) (layer F.Cu) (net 9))
 (segment (start 169.8756 60.7064) (end 169.8756 60.3) (width 0.2) (layer F.Cu) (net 9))
 (segment (start 171.5 61.25) (end 171.6892 61.25) (width 0.2) (layer F.Cu) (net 9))
 (segment (start 171.8056 61.3664) (end 171.8056 61.849) (width 0.2) (layer F.Cu) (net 9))
 (segment (start 171.6892 61.25) (end 171.8056 61.3664) (width 0.2) (layer F.Cu) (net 9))
 (segment (start 151.7396 61.5696) (end 151.7396 61.7982) (width 0.2) (layer F.Cu) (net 9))
 (segment (start 151.7396 61.7982) (end 152.0414 62.1) (width 0.2) (layer F.Cu) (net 9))
 (segment (start 152.0414 62.1) (end 152.5 62.1) (width 0.2) (layer F.Cu) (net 9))
 (segment (start 151.7396 61.087) (end 151.7396 61.0362) (width 0.2) (layer F.Cu) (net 9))
 (segment (start 154.4066 59.817) (end 154.8896 60.3) (width 0.2) (layer F.Cu) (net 9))
 (segment (start 152.9588 59.817) (end 154.4066 59.817) (width 0.2) (layer F.Cu) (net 9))
 (segment (start 151.7396 61.0362) (end 152.9588 59.817) (width 0.2) (layer F.Cu) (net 9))
 (segment (start 152.5 62.1) (end 152.27 62.1) (width 0.2) (layer F.Cu) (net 9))
 (segment (start 152.27 62.1) (end 151.7396 61.5696) (width 0.2) (layer F.Cu) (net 9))
 (segment (start 152.0698 61.087) (end 152.0952 61.0616) (width 0.2) (layer F.Cu) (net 9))
 (segment (start 151.7396 61.087) (end 152.0698 61.087) (width 0.2) (layer F.Cu) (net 9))
 (segment (start 151.7396 61.5696) (end 151.7396 61.087) (width 0.2) (layer F.Cu) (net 9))
 (segment (start 152.0952 61.0616) (end 152.0952 60.9092) (width 0.2) (layer F.Cu) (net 9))
 (segment (start 152.0952 60.9092) (end 152.0952 61.0616) (width 0.2) (layer F.Cu) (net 9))
 (segment (start 171.5 62.1) (end 171.5 61.9244) (width 0.5) (layer F.Cu) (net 9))
 (segment (start 171.5 61.9244) (end 169.8756 60.3) (width 0.5) (layer F.Cu) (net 9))
 (segment (start 152.5 62.1) (end 152.5 61.949) (width 0.5) (layer F.Cu) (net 9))
 (segment (start 152.5 61.949) (end 151.9936 61.4426) (width 0.5) (layer F.Cu) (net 9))
 (segment (start 152.4508 60.706) (end 152.4508 61.0492) (width 0.5) (layer F.Cu) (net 9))
 (segment (start 151.9936 61.1632) (end 152.0952 61.0616) (width 0.5) (layer F.Cu) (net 9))
 (segment (start 152.0952 61.0616) (end 152.4508 60.706) (width 0.5) (layer F.Cu) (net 9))
 (segment (start 151.9936 61.4426) (end 151.9936 61.1632) (width 0.5) (layer F.Cu) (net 9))
 (segment (start 171.5 62.1) (end 171.5 61.8236) (width 0.5) (layer F.Cu) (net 9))
 (segment (start 171.5 61.8236) (end 171.5 61.25) (width 0.5) (layer F.Cu) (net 9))
 (segment (start 152.45 61.05) (end 152.45 62.05) (width 0.5) (layer F.Cu) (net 9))
 (segment (start 153.2 60.3) (end 152.4508 61.0492) (width 1) (layer F.Cu) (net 9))
 (segment (start 154.8896 60.3) (end 153.2 60.3) (width 1) (layer F.Cu) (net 9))
 (segment (start 152.4508 61.0492) (end 152.45 61.05) (width 1) (layer F.Cu) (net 9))
 (segment (start 170.55 60.3) (end 169.8756 60.3) (width 1) (layer F.Cu) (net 9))
 (segment (start 169.8756 60.3) (end 154.8896 60.3) (width 1) (layer F.Cu) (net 9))
 (segment (start 171.5 61.25) (end 170.55 60.3) (width 1) (layer F.Cu) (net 9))
 (segment (start 152.45 62.05) (end 152.5 62.1) (width 0.5) (layer F.Cu) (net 9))
 (segment (start 171.75 65.1764) (end 171.75 66.25) (width 1) (layer F.Cu) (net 10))
 (segment (start 171.75 65.1764) (end 171.75 65.15) (width 0.5) (layer F.Cu) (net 10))
 (segment (start 190.5 65.9892) (end 190.5 65.4304) (width 1) (layer F.Cu) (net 10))
 (segment (start 190.5 64.9) (end 190.5 65.4304) (width 0.5) (layer F.Cu) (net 10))
 (segment (start 190.5 65.9892) (end 190.5 65.95) (width 0.5) (layer F.Cu) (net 10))
 (segment (start 172.1 66.6) (end 171.75 66.25) (width 1) (layer F.Cu) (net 10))
 (segment (start 189.85 66.6) (end 172.1 66.6) (width 1) (layer F.Cu) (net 10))
 (segment (start 190.5 65.95) (end 189.85 66.6) (width 1) (layer F.Cu) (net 10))
 (segment (start 171.75 65.15) (end 171.5 64.9) (width 0.5) (layer F.Cu) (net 10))
 (segment (start 190.55 61.45784) (end 190.66256 61.45784) (width 0.2) (layer F.Cu) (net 11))
 (segment (start 190.66256 61.45784) (end 191.05372 61.849) (width 0.2) (layer F.Cu) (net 11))
 (segment (start 190.55 61.45784) (end 190.55 61.45784) (width 0.2) (layer F.Cu) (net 11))
 (segment (start 190.55 61.45784) (end 190.44412 61.45784) (width 0.2) (layer F.Cu) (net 11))
 (segment (start 190.44412 61.45784) (end 190.06312 61.83884) (width 0.2) (layer F.Cu) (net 11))
 (segment (start 222.25 62.1) (end 222.25 61.5696) (width 0.5) (layer F.Cu) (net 11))
 (segment (start 222.25 61.5696) (end 222.0976 61.722) (width 0.5) (layer F.Cu) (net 11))
 (segment (start 221.9706 61.722) (end 222.25 61.722) (width 0.5) (layer F.Cu) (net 11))
 (segment (start 222.0976 61.722) (end 221.9706 61.722) (width 0.5) (layer F.Cu) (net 11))
 (segment (start 190.55 60.5028) (end 190.55 61.45784) (width 1) (layer F.Cu) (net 11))
 (segment (start 190.55 61.45784) (end 190.55 61.4672) (width 1) (layer F.Cu) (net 11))
 (segment (start 190.6016 61.5188) (end 190.55 61.5188) (width 1) (layer F.Cu) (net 11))
 (segment (start 190.55 61.4672) (end 190.6016 61.5188) (width 1) (layer F.Cu) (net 11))
 (segment (start 222.25 60.45) (end 222.25 61.722) (width 1) (layer F.Cu) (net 11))
 (segment (start 222.25 61.722) (end 222.25 61.5696) (width 1) (layer F.Cu) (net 11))
 (segment (start 190.55 60.4) (end 190.55 60.5028) (width 0.5) (layer F.Cu) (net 11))
 (segment (start 190.55 61.5188) (end 190.55 62.05) (width 0.5) (layer F.Cu) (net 11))
 (segment (start 191.65 59.3) (end 190.55 60.4) (width 1) (layer F.Cu) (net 11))
 (segment (start 221.1 59.3) (end 191.65 59.3) (width 1) (layer F.Cu) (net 11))
 (segment (start 222.25 60.45) (end 221.1 59.3) (width 1) (layer F.Cu) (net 11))
 (segment (start 190.55 62.05) (end 190.5 62.1) (width 0.5) (layer F.Cu) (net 11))
 (segment (start 131.9276 55.4228) (end 132.461 55.4228) (width 0.5) (layer F.Cu) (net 12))
 (segment (start 133.096 56.0578) (end 133.096 56.5912) (width 0.5) (layer F.Cu) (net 12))
 (segment (start 132.461 55.4228) (end 133.096 56.0578) (width 0.5) (layer F.Cu) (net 12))
 (segment (start 132.461 55.9562) (end 132.461 58.6486) (width 0.5) (layer F.Cu) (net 12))
 (segment (start 132.461 58.6486) (end 132.8166 59.0042) (width 0.5) (layer F.Cu) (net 12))
 (segment (start 132.7531 56.2483) (end 132.7531 58.4835) (width 0.5) (layer F.Cu) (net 12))
 (segment (start 132.7912 58.4708) (end 132.7912 58.4454) (width 0.5) (layer F.Cu) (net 12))
 (segment (start 132.7658 58.4708) (end 132.7912 58.4708) (width 0.5) (layer F.Cu) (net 12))
 (segment (start 132.7531 58.4835) (end 132.7658 58.4708) (width 0.5) (layer F.Cu) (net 12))
 (segment (start 133.096 58.166) (end 133.0706 58.166) (width 0.5) (layer F.Cu) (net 12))
 (segment (start 133.0706 58.166) (end 132.7912 58.4454) (width 0.5) (layer F.Cu) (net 12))
 (segment (start 133.1722 59.0042) (end 133.096 59.0042) (width 0.5) (layer F.Cu) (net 12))
 (segment (start 132.8166 59.0042) (end 133.1722 59.0042) (width 0.5) (layer F.Cu) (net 12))
 (segment (start 132.7912 58.4454) (end 132.5626 58.674) (width 0.5) (layer F.Cu) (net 12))
 (segment (start 132.5626 58.7502) (end 132.8166 59.0042) (width 0.5) (layer F.Cu) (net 12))
 (segment (start 132.5626 58.674) (end 132.5626 58.7502) (width 0.5) (layer F.Cu) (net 12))
 (segment (start 133.096 58.7502) (end 133.096 58.166) (width 0.5) (layer F.Cu) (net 12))
 (segment (start 133.096 58.166) (end 133.096 56.5912) (width 0.5) (layer F.Cu) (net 12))
 (segment (start 133.096 56.5912) (end 132.7531 56.2483) (width 0.5) (layer F.Cu) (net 12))
 (segment (start 132.7531 56.2483) (end 132.461 55.9562) (width 0.5) (layer F.Cu) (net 12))
 (segment (start 132.461 55.9562) (end 131.9276 55.4228) (width 0.5) (layer F.Cu) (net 12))
 (segment (start 133.096 58.928) (end 133.096 59.0042) (width 0.5) (layer F.Cu) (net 12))
 (segment (start 222.25 66.04) (end 222.25 65.4304) (width 1) (layer F.Cu) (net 12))
 (segment (start 222.25 64.9) (end 222.25 65.4304) (width 0.5) (layer F.Cu) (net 12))
 (segment (start 134.366 60.198) (end 133.096 58.928) (width 1) (layer F.Cu) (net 12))
 (segment (start 150.622 60.198) (end 134.366 60.198) (width 1) (layer F.Cu) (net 12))
 (segment (start 151.892 58.928) (end 150.622 60.198) (width 1) (layer F.Cu) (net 12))
 (segment (start 154.686 58.928) (end 151.892 58.928) (width 1) (layer F.Cu) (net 12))
 (segment (start 155.956 57.658) (end 154.686 58.928) (width 1) (layer F.Cu) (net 12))
 (segment (start 222.758 57.658) (end 155.956 57.658) (width 1) (layer F.Cu) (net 12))
 (segment (start 226.314 61.214) (end 222.758 57.658) (width 1) (layer F.Cu) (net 12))
 (segment (start 226.314 65.024) (end 226.314 61.214) (width 1) (layer F.Cu) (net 12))
 (segment (start 224.536 66.802) (end 226.314 65.024) (width 1) (layer F.Cu) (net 12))
 (segment (start 223.012 66.802) (end 224.536 66.802) (width 1) (layer F.Cu) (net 12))
 (segment (start 222.25 66.04) (end 223.012 66.802) (width 1) (layer F.Cu) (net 12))
 (segment (start 133.096 59.0042) (end 133.096 58.7502) (width 0.5) (layer F.Cu) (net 12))
 (segment (start 127.9652 55.88) (end 127.9652 55.9308) (width 0.5) (layer F.Cu) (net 12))
 (segment (start 127.9652 55.9308) (end 127.69 56.206) (width 0.5) (layer F.Cu) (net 12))
 (segment (start 127.69 56.206) (end 127.69 57.08) (width 0.5) (layer F.Cu) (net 12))
 (segment (start 131.9276 55.4228) (end 128.4224 55.4228) (width 0.5) (layer F.Cu) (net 12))
 (segment (start 128.4224 55.4228) (end 127.9652 55.88) (width 0.5) (layer F.Cu) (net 12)))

